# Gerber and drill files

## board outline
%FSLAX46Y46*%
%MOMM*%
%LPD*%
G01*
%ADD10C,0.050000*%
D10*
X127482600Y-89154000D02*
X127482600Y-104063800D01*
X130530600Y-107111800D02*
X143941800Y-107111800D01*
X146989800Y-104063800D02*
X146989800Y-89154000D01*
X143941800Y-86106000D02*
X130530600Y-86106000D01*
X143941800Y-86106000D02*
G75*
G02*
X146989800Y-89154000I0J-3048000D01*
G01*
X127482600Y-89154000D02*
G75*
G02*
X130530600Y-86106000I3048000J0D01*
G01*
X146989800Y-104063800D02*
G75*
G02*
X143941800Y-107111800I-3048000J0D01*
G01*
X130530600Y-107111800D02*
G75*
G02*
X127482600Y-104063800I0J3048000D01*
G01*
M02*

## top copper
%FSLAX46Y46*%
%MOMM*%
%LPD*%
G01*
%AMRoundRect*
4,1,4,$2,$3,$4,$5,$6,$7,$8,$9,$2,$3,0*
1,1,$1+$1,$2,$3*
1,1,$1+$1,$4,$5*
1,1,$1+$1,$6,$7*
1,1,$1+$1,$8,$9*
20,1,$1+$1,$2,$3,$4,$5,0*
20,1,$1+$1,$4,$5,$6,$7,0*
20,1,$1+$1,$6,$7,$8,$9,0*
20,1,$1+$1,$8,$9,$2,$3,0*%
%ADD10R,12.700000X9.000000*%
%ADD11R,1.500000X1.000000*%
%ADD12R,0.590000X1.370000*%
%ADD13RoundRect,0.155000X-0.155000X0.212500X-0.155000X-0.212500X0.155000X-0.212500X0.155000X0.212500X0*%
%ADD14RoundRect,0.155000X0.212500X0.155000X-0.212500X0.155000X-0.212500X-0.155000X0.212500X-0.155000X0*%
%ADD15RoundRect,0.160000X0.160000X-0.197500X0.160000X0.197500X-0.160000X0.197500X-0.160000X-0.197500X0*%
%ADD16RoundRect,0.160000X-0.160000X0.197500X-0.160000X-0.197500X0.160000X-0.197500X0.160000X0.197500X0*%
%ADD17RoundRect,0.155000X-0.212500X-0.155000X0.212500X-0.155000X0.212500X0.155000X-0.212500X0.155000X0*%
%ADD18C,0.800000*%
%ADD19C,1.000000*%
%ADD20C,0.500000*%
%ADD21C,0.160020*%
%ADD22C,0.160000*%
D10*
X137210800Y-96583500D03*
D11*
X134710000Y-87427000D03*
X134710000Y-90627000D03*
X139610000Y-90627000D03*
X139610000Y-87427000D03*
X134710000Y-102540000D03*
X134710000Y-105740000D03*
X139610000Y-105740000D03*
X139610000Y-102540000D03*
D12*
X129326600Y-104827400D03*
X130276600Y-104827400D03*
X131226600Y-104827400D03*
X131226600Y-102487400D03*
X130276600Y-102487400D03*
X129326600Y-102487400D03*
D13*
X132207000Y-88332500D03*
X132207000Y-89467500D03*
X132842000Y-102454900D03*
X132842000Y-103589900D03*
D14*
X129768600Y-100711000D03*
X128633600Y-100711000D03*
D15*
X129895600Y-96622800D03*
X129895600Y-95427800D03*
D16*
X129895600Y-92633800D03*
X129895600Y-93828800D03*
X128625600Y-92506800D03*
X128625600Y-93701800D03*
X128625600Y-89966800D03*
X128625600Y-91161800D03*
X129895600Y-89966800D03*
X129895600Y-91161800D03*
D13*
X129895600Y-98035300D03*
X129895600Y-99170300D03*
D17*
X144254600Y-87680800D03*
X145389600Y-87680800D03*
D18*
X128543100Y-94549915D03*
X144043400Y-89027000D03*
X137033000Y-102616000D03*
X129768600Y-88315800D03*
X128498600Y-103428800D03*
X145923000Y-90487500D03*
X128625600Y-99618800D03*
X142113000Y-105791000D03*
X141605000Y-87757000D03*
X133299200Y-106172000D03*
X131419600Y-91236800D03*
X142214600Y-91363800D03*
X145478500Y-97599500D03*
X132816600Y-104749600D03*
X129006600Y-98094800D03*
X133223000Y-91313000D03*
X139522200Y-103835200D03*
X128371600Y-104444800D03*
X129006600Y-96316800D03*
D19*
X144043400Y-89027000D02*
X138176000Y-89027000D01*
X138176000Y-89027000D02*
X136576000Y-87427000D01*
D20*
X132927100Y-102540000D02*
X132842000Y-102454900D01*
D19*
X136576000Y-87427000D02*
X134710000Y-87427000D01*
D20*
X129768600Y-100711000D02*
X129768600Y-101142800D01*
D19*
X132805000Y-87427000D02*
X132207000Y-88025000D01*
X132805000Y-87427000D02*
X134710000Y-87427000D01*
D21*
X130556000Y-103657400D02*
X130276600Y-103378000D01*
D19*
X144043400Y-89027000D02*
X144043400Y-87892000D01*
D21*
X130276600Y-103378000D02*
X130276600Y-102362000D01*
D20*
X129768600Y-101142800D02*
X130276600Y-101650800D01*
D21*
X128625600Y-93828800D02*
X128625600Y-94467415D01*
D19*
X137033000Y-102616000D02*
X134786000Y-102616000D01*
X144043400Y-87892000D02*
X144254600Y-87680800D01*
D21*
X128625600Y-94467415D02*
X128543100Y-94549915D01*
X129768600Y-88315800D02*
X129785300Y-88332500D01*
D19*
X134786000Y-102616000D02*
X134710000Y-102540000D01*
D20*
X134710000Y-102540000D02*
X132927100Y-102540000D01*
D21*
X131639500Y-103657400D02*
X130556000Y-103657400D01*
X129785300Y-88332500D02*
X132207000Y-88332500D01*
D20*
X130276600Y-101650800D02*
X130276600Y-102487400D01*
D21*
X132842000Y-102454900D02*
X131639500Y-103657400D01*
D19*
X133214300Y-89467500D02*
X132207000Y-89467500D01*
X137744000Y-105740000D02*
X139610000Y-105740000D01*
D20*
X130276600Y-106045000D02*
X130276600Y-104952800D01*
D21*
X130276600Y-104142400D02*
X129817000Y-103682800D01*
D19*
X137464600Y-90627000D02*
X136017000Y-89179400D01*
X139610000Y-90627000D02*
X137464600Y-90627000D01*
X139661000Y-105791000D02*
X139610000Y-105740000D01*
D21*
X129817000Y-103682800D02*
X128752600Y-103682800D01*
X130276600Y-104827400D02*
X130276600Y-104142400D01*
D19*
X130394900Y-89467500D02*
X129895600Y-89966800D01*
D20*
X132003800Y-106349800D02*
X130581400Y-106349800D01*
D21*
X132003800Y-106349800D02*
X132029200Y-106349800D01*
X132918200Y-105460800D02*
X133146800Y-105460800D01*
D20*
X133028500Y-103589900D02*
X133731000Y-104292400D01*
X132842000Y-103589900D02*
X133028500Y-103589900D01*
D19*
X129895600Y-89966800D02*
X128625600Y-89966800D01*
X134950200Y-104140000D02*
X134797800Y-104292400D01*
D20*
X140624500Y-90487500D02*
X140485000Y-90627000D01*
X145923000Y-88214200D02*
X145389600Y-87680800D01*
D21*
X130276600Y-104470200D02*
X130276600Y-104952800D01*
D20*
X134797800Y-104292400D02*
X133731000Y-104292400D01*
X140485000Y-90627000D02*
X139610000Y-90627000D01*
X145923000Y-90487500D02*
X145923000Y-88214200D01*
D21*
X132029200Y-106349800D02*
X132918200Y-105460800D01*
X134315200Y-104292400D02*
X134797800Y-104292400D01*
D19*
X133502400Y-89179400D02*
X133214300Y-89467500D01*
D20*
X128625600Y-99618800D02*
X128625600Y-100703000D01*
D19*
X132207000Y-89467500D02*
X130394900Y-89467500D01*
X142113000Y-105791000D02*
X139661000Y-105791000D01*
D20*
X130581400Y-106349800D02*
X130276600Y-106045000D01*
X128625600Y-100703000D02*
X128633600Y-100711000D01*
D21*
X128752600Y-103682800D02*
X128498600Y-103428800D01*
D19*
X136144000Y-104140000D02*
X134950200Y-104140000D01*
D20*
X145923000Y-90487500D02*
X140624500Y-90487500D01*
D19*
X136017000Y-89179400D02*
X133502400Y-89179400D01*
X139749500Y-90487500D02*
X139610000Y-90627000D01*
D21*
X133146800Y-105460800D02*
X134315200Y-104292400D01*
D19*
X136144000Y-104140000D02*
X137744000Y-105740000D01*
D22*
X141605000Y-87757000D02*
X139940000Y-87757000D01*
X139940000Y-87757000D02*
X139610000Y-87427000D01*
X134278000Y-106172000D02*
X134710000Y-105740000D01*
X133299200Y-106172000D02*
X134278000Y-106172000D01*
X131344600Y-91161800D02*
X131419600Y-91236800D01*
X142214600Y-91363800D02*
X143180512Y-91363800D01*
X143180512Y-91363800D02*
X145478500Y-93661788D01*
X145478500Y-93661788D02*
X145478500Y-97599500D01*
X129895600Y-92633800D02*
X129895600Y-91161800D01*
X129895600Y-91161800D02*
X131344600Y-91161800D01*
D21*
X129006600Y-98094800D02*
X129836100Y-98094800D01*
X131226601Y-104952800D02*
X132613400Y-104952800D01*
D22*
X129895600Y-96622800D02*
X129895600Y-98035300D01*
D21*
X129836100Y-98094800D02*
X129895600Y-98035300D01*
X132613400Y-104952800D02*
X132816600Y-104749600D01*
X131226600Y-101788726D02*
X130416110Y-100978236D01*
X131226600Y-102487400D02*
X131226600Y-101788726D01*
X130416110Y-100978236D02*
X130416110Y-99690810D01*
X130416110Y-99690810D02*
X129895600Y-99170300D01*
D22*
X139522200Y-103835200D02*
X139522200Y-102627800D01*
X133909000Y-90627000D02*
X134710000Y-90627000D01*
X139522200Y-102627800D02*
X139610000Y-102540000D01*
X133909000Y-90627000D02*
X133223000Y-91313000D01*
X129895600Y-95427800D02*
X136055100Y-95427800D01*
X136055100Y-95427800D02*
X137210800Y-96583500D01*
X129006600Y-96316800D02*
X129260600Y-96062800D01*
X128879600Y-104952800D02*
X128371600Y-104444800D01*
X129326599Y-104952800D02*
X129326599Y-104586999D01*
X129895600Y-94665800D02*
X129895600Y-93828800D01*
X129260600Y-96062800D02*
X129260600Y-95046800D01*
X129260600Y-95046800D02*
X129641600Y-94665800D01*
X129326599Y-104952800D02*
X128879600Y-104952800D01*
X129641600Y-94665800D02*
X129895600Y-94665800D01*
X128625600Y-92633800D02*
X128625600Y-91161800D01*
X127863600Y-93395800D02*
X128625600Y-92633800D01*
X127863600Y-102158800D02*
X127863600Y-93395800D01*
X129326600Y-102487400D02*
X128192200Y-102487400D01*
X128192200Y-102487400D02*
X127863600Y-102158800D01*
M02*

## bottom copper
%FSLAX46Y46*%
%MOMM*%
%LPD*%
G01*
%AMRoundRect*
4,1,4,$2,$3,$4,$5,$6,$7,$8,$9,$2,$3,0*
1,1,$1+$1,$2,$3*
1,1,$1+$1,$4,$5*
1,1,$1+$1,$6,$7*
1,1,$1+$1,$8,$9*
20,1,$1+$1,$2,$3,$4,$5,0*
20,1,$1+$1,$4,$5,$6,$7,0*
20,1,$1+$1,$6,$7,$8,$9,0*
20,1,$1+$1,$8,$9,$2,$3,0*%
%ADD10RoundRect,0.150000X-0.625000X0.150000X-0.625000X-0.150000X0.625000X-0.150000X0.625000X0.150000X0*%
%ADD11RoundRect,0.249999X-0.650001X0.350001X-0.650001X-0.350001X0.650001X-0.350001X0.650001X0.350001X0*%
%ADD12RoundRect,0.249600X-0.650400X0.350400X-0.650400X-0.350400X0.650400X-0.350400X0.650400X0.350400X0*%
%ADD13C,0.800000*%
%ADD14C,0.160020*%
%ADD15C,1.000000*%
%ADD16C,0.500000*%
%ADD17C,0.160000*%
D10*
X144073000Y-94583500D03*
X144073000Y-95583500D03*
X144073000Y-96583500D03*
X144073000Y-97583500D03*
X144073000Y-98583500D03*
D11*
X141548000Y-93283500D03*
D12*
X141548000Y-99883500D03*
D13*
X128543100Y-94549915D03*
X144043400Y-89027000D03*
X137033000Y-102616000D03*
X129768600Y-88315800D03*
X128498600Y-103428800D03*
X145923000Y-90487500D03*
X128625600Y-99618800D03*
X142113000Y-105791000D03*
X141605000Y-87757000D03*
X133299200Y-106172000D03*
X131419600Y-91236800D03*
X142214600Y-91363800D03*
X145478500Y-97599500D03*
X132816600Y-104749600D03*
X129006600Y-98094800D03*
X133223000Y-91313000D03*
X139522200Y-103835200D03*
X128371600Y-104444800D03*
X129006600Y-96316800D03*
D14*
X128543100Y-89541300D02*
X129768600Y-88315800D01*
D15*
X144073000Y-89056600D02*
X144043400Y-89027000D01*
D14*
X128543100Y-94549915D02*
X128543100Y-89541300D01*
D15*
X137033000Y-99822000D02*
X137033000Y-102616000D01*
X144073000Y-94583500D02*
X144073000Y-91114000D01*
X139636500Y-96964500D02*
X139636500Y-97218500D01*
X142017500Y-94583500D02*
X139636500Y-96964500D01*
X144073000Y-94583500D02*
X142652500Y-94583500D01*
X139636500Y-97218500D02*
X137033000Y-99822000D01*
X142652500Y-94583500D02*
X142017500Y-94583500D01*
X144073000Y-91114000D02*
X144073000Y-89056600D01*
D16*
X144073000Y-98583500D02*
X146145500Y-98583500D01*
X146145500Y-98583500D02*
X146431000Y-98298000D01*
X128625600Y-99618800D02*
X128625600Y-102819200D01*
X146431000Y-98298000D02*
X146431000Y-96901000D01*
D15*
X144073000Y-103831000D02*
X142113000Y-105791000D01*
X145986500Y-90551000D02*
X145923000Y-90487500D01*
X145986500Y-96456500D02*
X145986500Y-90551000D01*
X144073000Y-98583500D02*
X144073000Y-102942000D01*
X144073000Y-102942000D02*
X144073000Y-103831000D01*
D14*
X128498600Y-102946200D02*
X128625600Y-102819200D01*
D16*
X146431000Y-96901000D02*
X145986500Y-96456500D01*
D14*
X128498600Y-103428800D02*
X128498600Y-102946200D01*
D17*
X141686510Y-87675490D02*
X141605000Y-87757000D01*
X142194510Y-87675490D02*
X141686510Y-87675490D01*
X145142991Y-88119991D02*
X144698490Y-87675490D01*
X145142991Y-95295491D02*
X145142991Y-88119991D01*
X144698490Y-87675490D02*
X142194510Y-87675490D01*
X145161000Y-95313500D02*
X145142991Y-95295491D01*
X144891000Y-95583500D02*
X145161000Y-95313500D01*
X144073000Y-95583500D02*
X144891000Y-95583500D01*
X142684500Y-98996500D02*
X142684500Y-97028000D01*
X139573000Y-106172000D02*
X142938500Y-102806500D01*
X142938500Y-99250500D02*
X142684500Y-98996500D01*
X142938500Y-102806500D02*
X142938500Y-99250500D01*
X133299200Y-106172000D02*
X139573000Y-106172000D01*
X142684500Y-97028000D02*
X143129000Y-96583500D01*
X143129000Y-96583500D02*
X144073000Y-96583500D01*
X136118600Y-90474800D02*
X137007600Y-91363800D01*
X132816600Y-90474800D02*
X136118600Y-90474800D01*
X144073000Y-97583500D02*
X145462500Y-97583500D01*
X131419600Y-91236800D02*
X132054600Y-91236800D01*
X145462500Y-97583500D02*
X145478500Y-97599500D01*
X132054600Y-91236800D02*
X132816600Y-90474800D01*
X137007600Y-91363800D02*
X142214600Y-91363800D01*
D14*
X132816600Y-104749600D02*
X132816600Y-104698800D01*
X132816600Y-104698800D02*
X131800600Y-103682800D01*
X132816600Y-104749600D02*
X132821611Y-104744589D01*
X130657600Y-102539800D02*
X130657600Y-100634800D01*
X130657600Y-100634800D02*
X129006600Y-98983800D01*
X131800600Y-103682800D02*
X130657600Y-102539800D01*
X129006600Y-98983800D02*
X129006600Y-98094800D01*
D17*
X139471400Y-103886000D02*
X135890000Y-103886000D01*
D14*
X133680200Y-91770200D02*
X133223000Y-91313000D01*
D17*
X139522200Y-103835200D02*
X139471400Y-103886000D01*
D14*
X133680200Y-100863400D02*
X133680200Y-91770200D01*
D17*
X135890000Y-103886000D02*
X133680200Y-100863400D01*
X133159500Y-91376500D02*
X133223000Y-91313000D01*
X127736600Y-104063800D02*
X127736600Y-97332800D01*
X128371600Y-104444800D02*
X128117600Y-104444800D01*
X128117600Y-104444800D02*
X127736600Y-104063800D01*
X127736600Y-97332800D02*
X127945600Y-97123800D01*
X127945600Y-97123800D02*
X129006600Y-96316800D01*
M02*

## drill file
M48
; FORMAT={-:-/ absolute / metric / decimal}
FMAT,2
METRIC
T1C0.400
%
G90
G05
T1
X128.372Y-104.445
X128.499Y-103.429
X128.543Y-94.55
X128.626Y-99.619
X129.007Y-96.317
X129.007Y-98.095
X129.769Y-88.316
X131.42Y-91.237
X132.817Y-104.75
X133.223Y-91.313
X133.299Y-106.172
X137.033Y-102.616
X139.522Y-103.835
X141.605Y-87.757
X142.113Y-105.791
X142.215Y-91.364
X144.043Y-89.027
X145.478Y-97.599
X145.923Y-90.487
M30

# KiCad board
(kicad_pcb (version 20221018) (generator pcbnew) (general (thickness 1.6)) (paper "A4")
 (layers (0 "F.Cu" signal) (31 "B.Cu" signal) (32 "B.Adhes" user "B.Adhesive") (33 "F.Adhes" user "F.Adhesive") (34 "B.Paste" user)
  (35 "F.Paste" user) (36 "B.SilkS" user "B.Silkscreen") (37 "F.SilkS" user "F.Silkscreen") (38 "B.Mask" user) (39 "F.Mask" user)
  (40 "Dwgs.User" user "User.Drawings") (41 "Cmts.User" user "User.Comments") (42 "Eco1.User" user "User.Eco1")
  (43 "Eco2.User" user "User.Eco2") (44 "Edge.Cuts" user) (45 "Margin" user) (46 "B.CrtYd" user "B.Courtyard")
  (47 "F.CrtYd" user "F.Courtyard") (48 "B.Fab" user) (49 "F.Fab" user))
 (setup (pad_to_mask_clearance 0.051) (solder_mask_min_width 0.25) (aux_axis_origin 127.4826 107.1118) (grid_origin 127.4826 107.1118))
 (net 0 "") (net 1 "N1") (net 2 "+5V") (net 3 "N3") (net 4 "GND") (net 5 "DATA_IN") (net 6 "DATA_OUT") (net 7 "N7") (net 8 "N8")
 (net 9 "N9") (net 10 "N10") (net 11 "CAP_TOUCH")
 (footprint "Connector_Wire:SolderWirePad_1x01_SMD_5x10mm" (layer "F.Cu") (at 136.0805 96.647)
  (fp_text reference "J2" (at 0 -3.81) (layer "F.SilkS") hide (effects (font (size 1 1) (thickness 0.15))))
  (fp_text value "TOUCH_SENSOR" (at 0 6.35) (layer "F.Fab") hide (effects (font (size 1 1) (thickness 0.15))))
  (pad "1" smd rect (at 1.1303 -0.0635) (size 12.7 9) (layers "F.Cu" "F.Mask") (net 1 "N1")))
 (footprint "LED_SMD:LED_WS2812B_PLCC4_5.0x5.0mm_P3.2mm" (layer "F.Cu") (at 137.16 89.027)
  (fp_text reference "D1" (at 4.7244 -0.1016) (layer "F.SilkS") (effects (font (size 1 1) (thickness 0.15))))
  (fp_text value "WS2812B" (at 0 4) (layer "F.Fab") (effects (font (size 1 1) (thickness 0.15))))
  (pad "1" smd rect (at -2.45 -1.6) (size 1.5 1) (layers "F.Cu" "F.Paste" "F.Mask") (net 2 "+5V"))
  (pad "2" smd rect (at -2.45 1.6) (size 1.5 1) (layers "F.Cu" "F.Paste" "F.Mask") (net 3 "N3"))
  (pad "3" smd rect (at 2.45 1.6) (size 1.5 1) (layers "F.Cu" "F.Paste" "F.Mask") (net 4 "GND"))
  (pad "4" smd rect (at 2.45 -1.6) (size 1.5 1) (layers "F.Cu" "F.Paste" "F.Mask") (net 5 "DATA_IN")))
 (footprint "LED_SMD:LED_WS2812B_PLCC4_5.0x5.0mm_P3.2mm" (layer "F.Cu") (at 137.16 104.14)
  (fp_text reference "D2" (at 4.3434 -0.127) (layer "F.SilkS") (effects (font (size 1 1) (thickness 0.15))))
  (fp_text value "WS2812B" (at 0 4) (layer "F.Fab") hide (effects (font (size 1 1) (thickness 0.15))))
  (pad "1" smd rect (at -2.45 -1.6) (size 1.5 1) (layers "F.Cu" "F.Paste" "F.Mask") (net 2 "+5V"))
  (pad "2" smd rect (at -2.45 1.6) (size 1.5 1) (layers "F.Cu" "F.Paste" "F.Mask") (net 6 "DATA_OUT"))
  (pad "3" smd rect (at 2.45 1.6) (size 1.5 1) (layers "F.Cu" "F.Paste" "F.Mask") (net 4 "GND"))
  (pad "4" smd rect (at 2.45 -1.6) (size 1.5 1) (layers "F.Cu" "F.Paste" "F.Mask") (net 3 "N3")))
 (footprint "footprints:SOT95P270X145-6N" (layer "F.Cu") (at 130.2766 103.6574 90)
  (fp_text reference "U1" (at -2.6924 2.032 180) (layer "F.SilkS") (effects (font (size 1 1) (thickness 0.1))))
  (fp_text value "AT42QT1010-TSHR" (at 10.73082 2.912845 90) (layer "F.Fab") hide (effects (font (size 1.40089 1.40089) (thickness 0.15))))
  (pad "1" smd rect (at -1.17 -0.95 90) (size 1.37 0.59) (layers "F.Cu" "F.Paste" "F.Mask") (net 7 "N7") (solder_mask_margin 0.102))
  (pad "2" smd rect (at -1.17 0 90) (size 1.37 0.59) (layers "F.Cu" "F.Paste" "F.Mask") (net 4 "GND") (solder_mask_margin 0.102))
  (pad "3" smd rect (at -1.17 0.95 90) (size 1.37 0.59) (layers "F.Cu" "F.Paste" "F.Mask") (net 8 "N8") (solder_mask_margin 0.102))
  (pad "4" smd rect (at 1.17 0.95 90) (size 1.37 0.59) (layers "F.Cu" "F.Paste" "F.Mask") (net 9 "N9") (solder_mask_margin 0.102))
  (pad "5" smd rect (at 1.17 0 90) (size 1.37 0.59) (layers "F.Cu" "F.Paste" "F.Mask") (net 2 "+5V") (solder_mask_margin 0.102))
  (pad "6" smd rect (at 1.17 -0.95 90) (size 1.37 0.59) (layers "F.Cu" "F.Paste" "F.Mask") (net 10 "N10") (solder_mask_margin 0.102)))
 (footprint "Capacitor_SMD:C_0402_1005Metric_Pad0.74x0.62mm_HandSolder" (layer "F.Cu") (at 132.207 88.9 -90)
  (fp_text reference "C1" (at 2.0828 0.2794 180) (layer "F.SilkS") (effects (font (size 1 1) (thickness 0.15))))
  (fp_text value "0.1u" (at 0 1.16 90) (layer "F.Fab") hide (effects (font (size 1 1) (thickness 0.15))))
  (pad "1" smd roundrect (at -0.5675 0 270) (size 0.735 0.62) (layers "F.Cu" "F.Paste" "F.Mask") (roundrect_rratio 0.25) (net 2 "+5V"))
  (pad "2" smd roundrect (at 0.5675 0 270) (size 0.735 0.62) (layers "F.Cu" "F.Paste" "F.Mask") (roundrect_rratio 0.25) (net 4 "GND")))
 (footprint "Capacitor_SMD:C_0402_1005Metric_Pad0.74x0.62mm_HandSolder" (layer "F.Cu") (at 132.842 103.0224 -90)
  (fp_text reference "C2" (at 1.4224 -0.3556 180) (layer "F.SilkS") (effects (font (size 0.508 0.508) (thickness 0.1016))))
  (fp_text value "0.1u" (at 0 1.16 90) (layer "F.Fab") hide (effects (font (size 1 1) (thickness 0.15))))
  (pad "1" smd roundrect (at -0.5675 0 270) (size 0.735 0.62) (layers "F.Cu" "F.Paste" "F.Mask") (roundrect_rratio 0.25) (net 2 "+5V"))
  (pad "2" smd roundrect (at 0.5675 0 270) (size 0.735 0.62) (layers "F.Cu" "F.Paste" "F.Mask") (roundrect_rratio 0.25) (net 4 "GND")))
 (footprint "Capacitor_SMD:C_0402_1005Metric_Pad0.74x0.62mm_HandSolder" (layer "F.Cu") (at 129.2011 100.711 180)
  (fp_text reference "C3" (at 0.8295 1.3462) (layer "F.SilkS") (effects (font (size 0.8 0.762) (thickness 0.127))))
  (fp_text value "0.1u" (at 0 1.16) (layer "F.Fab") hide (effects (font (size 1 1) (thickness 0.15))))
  (pad "1" smd roundrect (at -0.5675 0 180) (size 0.735 0.62) (layers "F.Cu" "F.Paste" "F.Mask") (roundrect_rratio 0.25) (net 2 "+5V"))
  (pad "2" smd roundrect (at 0.5675 0 180) (size 0.735 0.62) (layers "F.Cu" "F.Paste" "F.Mask") (roundrect_rratio 0.25) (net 4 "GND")))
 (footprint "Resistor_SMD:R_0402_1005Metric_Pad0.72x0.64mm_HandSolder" (layer "F.Cu") (at 129.8956 96.0253 90)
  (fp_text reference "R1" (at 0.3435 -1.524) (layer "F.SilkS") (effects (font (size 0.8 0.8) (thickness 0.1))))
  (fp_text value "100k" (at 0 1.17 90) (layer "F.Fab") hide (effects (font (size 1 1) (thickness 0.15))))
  (pad "1" smd roundrect (at -0.5975 0 90) (size 0.715 0.64) (layers "F.Cu" "F.Paste" "F.Mask") (roundrect_rratio 0.25) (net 8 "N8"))
  (pad "2" smd roundrect (at 0.5975 0 90) (size 0.715 0.64) (layers "F.Cu" "F.Paste" "F.Mask") (roundrect_rratio 0.25) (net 1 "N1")))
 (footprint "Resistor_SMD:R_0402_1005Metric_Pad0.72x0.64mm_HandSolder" (layer "F.Cu") (at 129.8956 93.2313 -90)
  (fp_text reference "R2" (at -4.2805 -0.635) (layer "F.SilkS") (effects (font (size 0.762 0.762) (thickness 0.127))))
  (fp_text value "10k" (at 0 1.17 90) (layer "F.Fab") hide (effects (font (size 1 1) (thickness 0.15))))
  (pad "1" smd roundrect (at -0.5975 0 270) (size 0.715 0.64) (layers "F.Cu" "F.Paste" "F.Mask") (roundrect_rratio 0.25)
   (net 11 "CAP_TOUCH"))
  (pad "2" smd roundrect (at 0.5975 0 270) (size 0.715 0.64) (layers "F.Cu" "F.Paste" "F.Mask") (roundrect_rratio 0.25) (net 7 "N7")))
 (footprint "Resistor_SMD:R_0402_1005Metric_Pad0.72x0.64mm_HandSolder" (layer "F.Cu") (at 128.6256 93.1043 -90)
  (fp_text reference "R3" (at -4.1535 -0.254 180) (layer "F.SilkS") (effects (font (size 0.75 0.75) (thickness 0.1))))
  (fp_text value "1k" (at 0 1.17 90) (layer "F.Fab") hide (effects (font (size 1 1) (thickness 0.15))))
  (pad "1" smd roundrect (at -0.5975 0 270) (size 0.715 0.64) (layers "F.Cu" "F.Paste" "F.Mask") (roundrect_rratio 0.25) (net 10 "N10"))
  (pad "2" smd roundrect (at 0.5975 0 270) (size 0.715 0.64) (layers "F.Cu" "F.Paste" "F.Mask") (roundrect_rratio 0.25) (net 2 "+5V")))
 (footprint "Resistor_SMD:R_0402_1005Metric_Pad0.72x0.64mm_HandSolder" (layer "F.Cu") (at 128.6256 90.5643 -90)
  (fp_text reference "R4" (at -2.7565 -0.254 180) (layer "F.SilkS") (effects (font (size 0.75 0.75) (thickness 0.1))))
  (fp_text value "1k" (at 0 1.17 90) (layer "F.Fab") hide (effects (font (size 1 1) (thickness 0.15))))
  (pad "1" smd roundrect (at -0.5975 0 270) (size 0.715 0.64) (layers "F.Cu" "F.Paste" "F.Mask") (roundrect_rratio 0.25) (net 4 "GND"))
  (pad "2" smd roundrect (at 0.5975 0 270) (size 0.715 0.64) (layers "F.Cu" "F.Paste" "F.Mask") (roundrect_rratio 0.25) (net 10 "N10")))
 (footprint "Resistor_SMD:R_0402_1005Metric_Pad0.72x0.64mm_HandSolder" (layer "F.Cu") (at 129.8956 90.5643 -90)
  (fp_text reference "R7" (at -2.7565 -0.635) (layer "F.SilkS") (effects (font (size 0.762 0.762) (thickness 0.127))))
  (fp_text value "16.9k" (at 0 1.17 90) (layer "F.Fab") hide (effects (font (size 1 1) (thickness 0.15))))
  (pad "1" smd roundrect (at -0.5975 0 270) (size 0.715 0.64) (layers "F.Cu" "F.Paste" "F.Mask") (roundrect_rratio 0.25) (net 4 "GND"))
  (pad "2" smd roundrect (at 0.5975 0 270) (size 0.715 0.64) (layers "F.Cu" "F.Paste" "F.Mask") (roundrect_rratio 0.25) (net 11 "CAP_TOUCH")))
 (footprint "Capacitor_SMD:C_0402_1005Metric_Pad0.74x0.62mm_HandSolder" (layer "F.Cu") (at 129.8956 98.6028 -90)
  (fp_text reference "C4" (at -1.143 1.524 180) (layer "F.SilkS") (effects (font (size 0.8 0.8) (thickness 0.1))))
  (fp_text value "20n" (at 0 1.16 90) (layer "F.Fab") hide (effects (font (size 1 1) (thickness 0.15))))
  (pad "1" smd roundrect (at -0.5675 0 270) (size 0.735 0.62) (layers "F.Cu" "F.Paste" "F.Mask") (roundrect_rratio 0.25) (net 8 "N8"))
  (pad "2" smd roundrect (at 0.5675 0 270) (size 0.735 0.62) (layers "F.Cu" "F.Paste" "F.Mask") (roundrect_rratio 0.25) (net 9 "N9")))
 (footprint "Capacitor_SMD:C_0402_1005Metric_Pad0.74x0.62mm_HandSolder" (layer "F.Cu") (at 144.8221 87.6808)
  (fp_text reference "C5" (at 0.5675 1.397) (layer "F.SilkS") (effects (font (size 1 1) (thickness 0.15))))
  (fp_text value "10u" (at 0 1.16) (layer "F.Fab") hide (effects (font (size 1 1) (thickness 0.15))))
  (pad "1" smd roundrect (at -0.5675 0) (size 0.735 0.62) (layers "F.Cu" "F.Paste" "F.Mask") (roundrect_rratio 0.25) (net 2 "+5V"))
  (pad "2" smd roundrect (at 0.5675 0) (size 0.735 0.62) (layers "F.Cu" "F.Paste" "F.Mask") (roundrect_rratio 0.25) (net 4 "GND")))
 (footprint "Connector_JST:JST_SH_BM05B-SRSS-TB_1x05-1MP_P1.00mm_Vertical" (layer "B.Cu") (at 142.748 96.5835 -90)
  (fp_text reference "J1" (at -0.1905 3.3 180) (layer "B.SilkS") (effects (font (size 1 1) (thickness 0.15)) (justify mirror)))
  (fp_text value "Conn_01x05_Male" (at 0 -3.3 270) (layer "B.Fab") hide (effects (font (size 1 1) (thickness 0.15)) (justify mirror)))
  (pad "1" smd roundrect (at -2 -1.325 270) (size 0.6 1.55) (layers "B.Cu" "B.Mask") (roundrect_rratio 0.25) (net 2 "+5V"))
  (pad "2" smd roundrect (at -1 -1.325 270) (size 0.6 1.55) (layers "B.Cu" "B.Mask") (roundrect_rratio 0.25) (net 5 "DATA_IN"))
  (pad "3" smd roundrect (at 0 -1.325 270) (size 0.6 1.55) (layers "B.Cu" "B.Mask") (roundrect_rratio 0.25) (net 6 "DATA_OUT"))
  (pad "4" smd roundrect (at 1 -1.325 270) (size 0.6 1.55) (layers "B.Cu" "B.Mask") (roundrect_rratio 0.25) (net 11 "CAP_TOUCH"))
  (pad "5" smd roundrect (at 2 -1.325 270) (size 0.6 1.55) (layers "B.Cu" "B.Mask") (roundrect_rratio 0.25) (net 4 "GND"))
  (pad "MP" smd roundrect (at -3.3 1.2 270) (size 1.2 1.8) (layers "B.Cu" "B.Paste" "B.Mask") (roundrect_rratio 0.2083325))
  (pad "MP" smd roundrect (at 3.3 1.2 270) (size 1.2 1.8) (layers "B.Cu" "B.Mask") (roundrect_rratio 0.208)))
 (gr_line (start 127.4826 89.154) (end 127.4826 104.0638) (stroke (width 0.05) (type solid)) (layer "Edge.Cuts"))
 (gr_line (start 130.5306 107.1118) (end 143.9418 107.1118) (stroke (width 0.05) (type solid)) (layer "Edge.Cuts"))
 (gr_line (start 146.9898 104.0638) (end 146.9898 89.154) (stroke (width 0.05) (type solid)) (layer "Edge.Cuts"))
 (gr_line (start 143.9418 86.106) (end 130.5306 86.106) (stroke (width 0.05) (type solid)) (layer "Edge.Cuts"))
 (gr_arc (start 143.9418 86.106) (mid 146.097061 86.998739) (end 146.9898 89.154) (stroke (width 0.05) (type solid)) (layer "Edge.Cuts"))
 (gr_arc (start 127.4826 89.154) (mid 128.375339 86.998739) (end 130.5306 86.106) (stroke (width 0.05) (type solid)) (layer "Edge.Cuts"))
 (gr_arc (start 146.9898 104.0638) (mid 146.097061 106.219061) (end 143.9418 107.1118) (stroke (width 0.05) (type solid))
  (layer "Edge.Cuts"))
 (gr_arc (start 130.5306 107.1118) (mid 128.375339 106.219061) (end 127.4826 104.0638) (stroke (width 0.05) (type solid))
  (layer "Edge.Cuts"))
 (segment (start 144.0434 89.027) (end 138.176 89.027) (width 1) (layer "F.Cu") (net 2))
 (segment (start 138.176 89.027) (end 136.576 87.427) (width 1) (layer "F.Cu") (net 2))
 (segment (start 132.9271 102.54) (end 132.842 102.4549) (width 0.5) (layer "F.Cu") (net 2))
 (segment (start 136.576 87.427) (end 134.71 87.427) (width 1) (layer "F.Cu") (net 2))
 (segment (start 129.7686 100.711) (end 129.7686 101.1428) (width 0.5) (layer "F.Cu") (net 2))
 (segment (start 132.805 87.427) (end 132.207 88.025) (width 1) (layer "F.Cu") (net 2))
 (segment (start 132.805 87.427) (end 134.71 87.427) (width 1) (layer "F.Cu") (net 2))
 (segment (start 130.556 103.6574) (end 130.2766 103.378) (width 0.16002) (layer "F.Cu") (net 2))
 (segment (start 144.0434 89.027) (end 144.0434 87.892) (width 1) (layer "F.Cu") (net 2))
 (segment (start 130.2766 103.378) (end 130.2766 102.362) (width 0.16002) (layer "F.Cu") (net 2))
 (segment (start 129.7686 101.1428) (end 130.2766 101.6508) (width 0.5) (layer "F.Cu") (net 2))
 (segment (start 128.6256 93.8288) (end 128.6256 94.467415) (width 0.16002) (layer "F.Cu") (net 2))
 (segment (start 137.033 102.616) (end 134.786 102.616) (width 1) (layer "F.Cu") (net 2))
 (segment (start 144.0434 87.892) (end 144.2546 87.6808) (width 1) (layer "F.Cu") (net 2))
 (segment (start 128.6256 94.467415) (end 128.5431 94.549915) (width 0.16002) (layer "F.Cu") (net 2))
 (segment (start 129.7686 88.3158) (end 129.7853 88.3325) (width 0.16002) (layer "F.Cu") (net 2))
 (segment (start 134.786 102.616) (end 134.71 102.54) (width 1) (layer "F.Cu") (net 2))
 (segment (start 134.71 102.54) (end 132.9271 102.54) (width 0.5) (layer "F.Cu") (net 2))
 (segment (start 131.6395 103.6574) (end 130.556 103.6574) (width 0.16002) (layer "F.Cu") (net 2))
 (segment (start 129.7853 88.3325) (end 132.207 88.3325) (width 0.16002) (layer "F.Cu") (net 2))
 (segment (start 130.2766 101.6508) (end 130.2766 102.4874) (width 0.5) (layer "F.Cu") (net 2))
 (segment (start 132.842 102.4549) (end 131.6395 103.6574) (width 0.16002) (layer "F.Cu") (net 2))
 (via (at 128.5431 94.549915) (size 0.8) (drill 0.4) (layers "F.Cu" "B.Cu") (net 2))
 (via (at 144.0434 89.027) (size 0.8) (drill 0.4) (layers "F.Cu" "B.Cu") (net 2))
 (via (at 137.033 102.616) (size 0.8) (drill 0.4) (layers "F.Cu" "B.Cu") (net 2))
 (via (at 129.7686 88.3158) (size 0.8) (drill 0.4) (layers "F.Cu" "B.Cu") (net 2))
 (segment (start 128.5431 89.5413) (end 129.7686 88.3158) (width 0.16002) (layer "B.Cu") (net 2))
 (segment (start 144.073 89.0566) (end 144.0434 89.027) (width 1) (layer "B.Cu") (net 2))
 (segment (start 128.5431 94.549915) (end 128.5431 89.5413) (width 0.16002) (layer "B.Cu") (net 2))
 (segment (start 137.033 99.822) (end 137.033 102.616) (width 1) (layer "B.Cu") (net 2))
 (segment (start 144.073 94.5835) (end 144.073 91.114) (width 1) (layer "B.Cu") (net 2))
 (segment (start 139.6365 96.9645) (end 139.6365 97.2185) (width 1) (layer "B.Cu") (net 2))
 (segment (start 142.0175 94.5835) (end 139.6365 96.9645) (width 1) (layer "B.Cu") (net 2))
 (segment (start 144.073 94.5835) (end 142.6525 94.5835) (width 1) (layer "B.Cu") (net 2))
 (segment (start 139.6365 97.2185) (end 137.033 99.822) (width 1) (layer "B.Cu") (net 2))
 (segment (start 142.6525 94.5835) (end 142.0175 94.5835) (width 1) (layer "B.Cu") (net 2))
 (segment (start 144.073 91.114) (end 144.073 89.0566) (width 1) (layer "B.Cu") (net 2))
 (segment (start 133.2143 89.4675) (end 132.207 89.4675) (width 1) (layer "F.Cu") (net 4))
 (segment (start 137.744 105.74) (end 139.61 105.74) (width 1) (layer "F.Cu") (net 4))
 (segment (start 130.2766 106.045) (end 130.2766 104.9528) (width 0.5) (layer "F.Cu") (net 4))
 (segment (start 130.2766 104.1424) (end 129.817 103.6828) (width 0.16002) (layer "F.Cu") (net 4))
 (segment (start 137.4646 90.627) (end 136.017 89.1794) (width 1) (layer "F.Cu") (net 4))
 (segment (start 139.61 90.627) (end 137.4646 90.627) (width 1) (layer "F.Cu") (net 4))
 (segment (start 139.661 105.791) (end 139.61 105.74) (width 1) (layer "F.Cu") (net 4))
 (segment (start 129.817 103.6828) (end 128.7526 103.6828) (width 0.16002) (layer "F.Cu") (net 4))
 (segment (start 130.2766 104.8274) (end 130.2766 104.1424) (width 0.16002) (layer "F.Cu") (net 4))
 (segment (start 130.3949 89.4675) (end 129.8956 89.9668) (width 1) (layer "F.Cu") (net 4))
 (segment (start 132.0038 106.3498) (end 130.5814 106.3498) (width 0.5) (layer "F.Cu") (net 4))
 (segment (start 132.0038 106.3498) (end 132.0292 106.3498) (width 0.16002) (layer "F.Cu") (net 4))
 (segment (start 132.9182 105.4608) (end 133.1468 105.4608) (width 0.16002) (layer "F.Cu") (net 4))
 (segment (start 133.0285 103.5899) (end 133.731 104.2924) (width 0.5) (layer "F.Cu") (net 4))
 (segment (start 132.842 103.5899) (end 133.0285 103.5899) (width 0.5) (layer "F.Cu") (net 4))
 (segment (start 129.8956 89.9668) (end 128.6256 89.9668) (width 1) (layer "F.Cu") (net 4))
 (segment (start 134.9502 104.14) (end 134.7978 104.2924) (width 1) (layer "F.Cu") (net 4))
 (segment (start 140.6245 90.4875) (end 140.485 90.627) (width 0.5) (layer "F.Cu") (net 4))
 (segment (start 145.923 88.2142) (end 145.3896 87.6808) (width 0.5) (layer "F.Cu") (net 4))
 (segment (start 130.2766 104.4702) (end 130.2766 104.9528) (width 0.16002) (layer "F.Cu") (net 4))
 (segment (start 134.7978 104.2924) (end 133.731 104.2924) (width 0.5) (layer "F.Cu") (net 4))
 (segment (start 140.485 90.627) (end 139.61 90.627) (width 0.5) (layer "F.Cu") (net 4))
 (segment (start 145.923 90.4875) (end 145.923 88.2142) (width 0.5) (layer "F.Cu") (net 4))
 (segment (start 132.0292 106.3498) (end 132.9182 105.4608) (width 0.16002) (layer "F.Cu") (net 4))
 (segment (start 134.3152 104.2924) (end 134.7978 104.2924) (width 0.16002) (layer "F.Cu") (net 4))
 (segment (start 133.5024 89.1794) (end 133.2143 89.4675) (width 1) (layer "F.Cu") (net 4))
 (segment (start 128.6256 99.6188) (end 128.6256 100.703) (width 0.5) (layer "F.Cu") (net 4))
 (segment (start 132.207 89.4675) (end 130.3949 89.4675) (width 1) (layer "F.Cu") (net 4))
 (segment (start 142.113 105.791) (end 139.661 105.791) (width 1) (layer "F.Cu") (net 4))
 (segment (start 130.5814 106.3498) (end 130.2766 106.045) (width 0.5) (layer "F.Cu") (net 4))
 (segment (start 128.6256 100.703) (end 128.6336 100.711) (width 0.5) (layer "F.Cu") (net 4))
 (segment (start 128.7526 103.6828) (end 128.4986 103.4288) (width 0.16002) (layer "F.Cu") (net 4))
 (segment (start 136.144 104.14) (end 134.9502 104.14) (width 1) (layer "F.Cu") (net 4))
 (segment (start 145.923 90.4875) (end 140.6245 90.4875) (width 0.5) (layer "F.Cu") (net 4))
 (segment (start 136.017 89.1794) (end 133.5024 89.1794) (width 1) (layer "F.Cu") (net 4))
 (segment (start 139.7495 90.4875) (end 139.61 90.627) (width 1) (layer "F.Cu") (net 4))
 (segment (start 133.1468 105.4608) (end 134.3152 104.2924) (width 0.16002) (layer "F.Cu") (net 4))
 (segment (start 136.144 104.14) (end 137.744 105.74) (width 1) (layer "F.Cu") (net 4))
 (via (at 128.4986 103.4288) (size 0.8) (drill 0.4) (layers "F.Cu" "B.Cu") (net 4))
 (via (at 145.923 90.4875) (size 0.8) (drill 0.4) (layers "F.Cu" "B.Cu") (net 4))
 (via (at 128.6256 99.6188) (size 0.8) (drill 0.4) (layers "F.Cu" "B.Cu") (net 4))
 (via (at 142.113 105.791) (size 0.8) (drill 0.4) (layers "F.Cu" "B.Cu") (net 4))
 (segment (start 144.073 98.5835) (end 146.1455 98.5835) (width 0.5) (layer "B.Cu") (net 4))
 (segment (start 146.1455 98.5835) (end 146.431 98.298) (width 0.5) (layer "B.Cu") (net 4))
 (segment (start 128.6256 99.6188) (end 128.6256 102.8192) (width 0.5) (layer "B.Cu") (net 4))
 (segment (start 146.431 98.298) (end 146.431 96.901) (width 0.5) (layer "B.Cu") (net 4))
 (segment (start 144.073 103.831) (end 142.113 105.791) (width 1) (layer "B.Cu") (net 4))
 (segment (start 145.9865 90.551) (end 145.923 90.4875) (width 1) (layer "B.Cu") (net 4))
 (segment (start 145.9865 96.4565) (end 145.9865 90.551) (width 1) (layer "B.Cu") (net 4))
 (segment (start 144.073 98.5835) (end 144.073 102.942) (width 1) (layer "B.Cu") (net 4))
 (segment (start 144.073 102.942) (end 144.073 103.831) (width 1) (layer "B.Cu") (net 4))
 (segment (start 128.4986 102.9462) (end 128.6256 102.8192) (width 0.16002) (layer "B.Cu") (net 4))
 (segment (start 146.431 96.901) (end 145.9865 96.4565) (width 0.5) (layer "B.Cu") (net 4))
 (segment (start 128.4986 103.4288) (end 128.4986 102.9462) (width 0.16002) (layer "B.Cu") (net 4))
 (segment (start 141.605 87.757) (end 139.94 87.757) (width 0.16) (layer "F.Cu") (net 5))
 (segment (start 139.94 87.757) (end 139.61 87.427) (width 0.16) (layer "F.Cu") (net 5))
 (via (at 141.605 87.757) (size 0.8) (drill 0.4) (layers "F.Cu" "B.Cu") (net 5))
 (segment (start 141.68651 87.67549) (end 141.605 87.757) (width 0.16) (layer "B.Cu") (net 5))
 (segment (start 142.19451 87.67549) (end 141.68651 87.67549) (width 0.16) (layer "B.Cu") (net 5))
 (segment (start 145.142991 88.119991) (end 144.69849 87.67549) (width 0.16) (layer "B.Cu") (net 5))
 (segment (start 145.142991 95.295491) (end 145.142991 88.119991) (width 0.16) (layer "B.Cu") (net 5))
 (segment (start 144.69849 87.67549) (end 142.19451 87.67549) (width 0.16) (layer "B.Cu") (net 5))
 (segment (start 145.161 95.3135) (end 145.142991 95.295491) (width 0.16) (layer "B.Cu") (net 5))
 (segment (start 144.891 95.5835) (end 145.161 95.3135) (width 0.16) (layer "B.Cu") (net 5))
 (segment (start 144.073 95.5835) (end 144.891 95.5835) (width 0.16) (layer "B.Cu") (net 5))
 (segment (start 134.278 106.172) (end 134.71 105.74) (width 0.16) (layer "F.Cu") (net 6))
 (segment (start 133.2992 106.172) (end 134.278 106.172) (width 0.16) (layer "F.Cu") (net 6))
 (via (at 133.2992 106.172) (size 0.8) (drill 0.4) (layers "F.Cu" "B.Cu") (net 6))
 (segment (start 142.6845 98.9965) (end 142.6845 97.028) (width 0.16) (layer "B.Cu") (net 6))
 (segment (start 139.573 106.172) (end 142.9385 102.8065) (width 0.16) (layer "B.Cu") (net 6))
 (segment (start 142.9385 99.2505) (end 142.6845 98.9965) (width 0.16) (layer "B.Cu") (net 6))
 (segment (start 142.9385 102.8065) (end 142.9385 99.2505) (width 0.16) (layer "B.Cu") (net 6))
 (segment (start 133.2992 106.172) (end 139.573 106.172) (width 0.16) (layer "B.Cu") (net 6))
 (segment (start 142.6845 97.028) (end 143.129 96.5835) (width 0.16) (layer "B.Cu") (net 6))
 (segment (start 143.129 96.5835) (end 144.073 96.5835) (width 0.16) (layer "B.Cu") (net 6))
 (segment (start 131.3446 91.1618) (end 131.4196 91.2368) (width 0.16) (layer "F.Cu") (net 11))
 (segment (start 142.2146 91.3638) (end 143.180512 91.3638) (width 0.16) (layer "F.Cu") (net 11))
 (segment (start 143.180512 91.3638) (end 145.4785 93.661788) (width 0.16) (layer "F.Cu") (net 11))
 (segment (start 145.4785 93.661788) (end 145.4785 97.5995) (width 0.16) (layer "F.Cu") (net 11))
 (segment (start 129.8956 92.6338) (end 129.8956 91.1618) (width 0.16) (layer "F.Cu") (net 11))
 (segment (start 129.8956 91.1618) (end 131.3446 91.1618) (width 0.16) (layer "F.Cu") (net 11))
 (via (at 131.4196 91.2368) (size 0.8) (drill 0.4) (layers "F.Cu" "B.Cu") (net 11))
 (via (at 142.2146 91.3638) (size 0.8) (drill 0.4) (layers "F.Cu" "B.Cu") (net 11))
 (via (at 145.4785 97.5995) (size 0.8) (drill 0.4) (layers "F.Cu" "B.Cu") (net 11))
 (segment (start 136.1186 90.4748) (end 137.0076 91.3638) (width 0.16) (layer "B.Cu") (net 11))
 (segment (start 132.8166 90.4748) (end 136.1186 90.4748) (width 0.16) (layer "B.Cu") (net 11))
 (segment (start 144.073 97.5835) (end 145.4625 97.5835) (width 0.16) (layer "B.Cu") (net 11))
 (segment (start 131.4196 91.2368) (end 132.0546 91.2368) (width 0.16) (layer "B.Cu") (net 11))
 (segment (start 145.4625 97.5835) (end 145.4785 97.5995) (width 0.16) (layer "B.Cu") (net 11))
 (segment (start 132.0546 91.2368) (end 132.8166 90.4748) (width 0.16) (layer "B.Cu") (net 11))
 (segment (start 137.0076 91.3638) (end 142.2146 91.3638) (width 0.16) (layer "B.Cu") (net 11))
 (segment (start 129.0066 98.0948) (end 129.8361 98.0948) (width 0.16002) (layer "F.Cu") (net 8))
 (segment (start 131.226601 104.9528) (end 132.6134 104.9528) (width 0.16002) (layer "F.Cu") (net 8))
 (segment (start 129.8956 96.6228) (end 129.8956 98.0353) (width 0.16) (layer "F.Cu") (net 8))
 (segment (start 129.8361 98.0948) (end 129.8956 98.0353) (width 0.16002) (layer "F.Cu") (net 8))
 (segment (start 132.6134 104.9528) (end 132.8166 104.7496) (width 0.16002) (layer "F.Cu") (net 8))
 (via (at 132.8166 104.7496) (size 0.8) (drill 0.4) (layers "F.Cu" "B.Cu") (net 8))
 (via (at 129.0066 98.0948) (size 0.8) (drill 0.4) (layers "F.Cu" "B.Cu") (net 8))
 (segment (start 132.8166 104.7496) (end 132.8166 104.6988) (width 0.16002) (layer "B.Cu") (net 8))
 (segment (start 132.8166 104.6988) (end 131.8006 103.6828) (width 0.16002) (layer "B.Cu") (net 8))
 (segment (start 132.8166 104.7496) (end 132.821611 104.744589) (width 0.16002) (layer "B.Cu") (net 8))
 (segment (start 130.6576 102.5398) (end 130.6576 100.6348) (width 0.16002) (layer "B.Cu") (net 8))
 (segment (start 130.6576 100.6348) (end 129.0066 98.9838) (width 0.16002) (layer "B.Cu") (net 8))
 (segment (start 131.8006 103.6828) (end 130.6576 102.5398) (width 0.16002) (layer "B.Cu") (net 8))
 (segment (start 129.0066 98.9838) (end 129.0066 98.0948) (width 0.16002) (layer "B.Cu") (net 8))
 (segment (start 131.2266 101.788726) (end 130.41611 100.978236) (width 0.16002) (layer "F.Cu") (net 9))
 (segment (start 131.2266 102.4874) (end 131.2266 101.788726) (width 0.16002) (layer "F.Cu") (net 9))
 (segment (start 130.41611 100.978236) (end 130.41611 99.69081) (width 0.16002) (layer "F.Cu") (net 9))
 (segment (start 130.41611 99.69081) (end 129.8956 99.1703) (width 0.16002) (layer "F.Cu") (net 9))
 (segment (start 139.5222 103.8352) (end 139.5222 102.6278) (width 0.16) (layer "F.Cu") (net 3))
 (segment (start 133.909 90.627) (end 134.71 90.627) (width 0.16) (layer "F.Cu") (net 3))
 (segment (start 139.5222 102.6278) (end 139.61 102.54) (width 0.16) (layer "F.Cu") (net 3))
 (segment (start 133.909 90.627) (end 133.223 91.313) (width 0.16) (layer "F.Cu") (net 3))
 (via (at 133.223 91.313) (size 0.8) (drill 0.4) (layers "F.Cu" "B.Cu") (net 3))
 (via (at 139.5222 103.8352) (size 0.8) (drill 0.4) (layers "F.Cu" "B.Cu") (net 3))
 (segment (start 139.4714 103.886) (end 135.89 103.886) (width 0.16) (layer "B.Cu") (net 3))
 (segment (start 133.6802 91.7702) (end 133.223 91.313) (width 0.16002) (layer "B.Cu") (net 3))
 (segment (start 139.5222 103.8352) (end 139.4714 103.886) (width 0.16) (layer "B.Cu") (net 3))
 (segment (start 133.6802 100.8634) (end 133.6802 91.7702) (width 0.16002) (layer "B.Cu") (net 3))
 (segment (start 135.89 103.886) (end 133.6802 100.8634) (width 0.16) (layer "B.Cu") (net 3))
 (segment (start 133.1595 91.3765) (end 133.223 91.313) (width 0.16) (layer "B.Cu") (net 3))
 (segment (start 129.8956 95.4278) (end 136.0551 95.4278) (width 0.16) (layer "F.Cu") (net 1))
 (segment (start 136.0551 95.4278) (end 137.2108 96.5835) (width 0.16) (layer "F.Cu") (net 1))
 (segment (start 129.0066 96.3168) (end 129.2606 96.0628) (width 0.16) (layer "F.Cu") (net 7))
 (segment (start 128.8796 104.9528) (end 128.3716 104.4448) (width 0.16) (layer "F.Cu") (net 7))
 (segment (start 129.326599 104.9528) (end 129.326599 104.586999) (width 0.16) (layer "F.Cu") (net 7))
 (segment (start 129.8956 94.6658) (end 129.8956 93.8288) (width 0.16) (layer "F.Cu") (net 7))
 (segment (start 129.2606 96.0628) (end 129.2606 95.0468) (width 0.16) (layer "F.Cu") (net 7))
 (segment (start 129.2606 95.0468) (end 129.6416 94.6658) (width 0.16) (layer "F.Cu") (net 7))
 (segment (start 129.326599 104.9528) (end 128.8796 104.9528) (width 0.16) (layer "F.Cu") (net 7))
 (segment (start 129.6416 94.6658) (end 129.8956 94.6658) (width 0.16) (layer "F.Cu") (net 7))
 (via (at 128.3716 104.4448) (size 0.8) (drill 0.4) (layers "F.Cu" "B.Cu") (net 7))
 (via (at 129.0066 96.3168) (size 0.8) (drill 0.4) (layers "F.Cu" "B.Cu") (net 7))
 (segment (start 127.7366 104.0638) (end 127.7366 97.3328) (width 0.16) (layer "B.Cu") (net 7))
 (segment (start 128.3716 104.4448) (end 128.1176 104.4448) (width 0.16) (layer "B.Cu") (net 7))
 (segment (start 128.1176 104.4448) (end 127.7366 104.0638) (width 0.16) (layer "B.Cu") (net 7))
 (segment (start 127.7366 97.3328) (end 127.9456 97.1238) (width 0.16) (layer "B.Cu") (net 7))
 (segment (start 127.9456 97.1238) (end 129.0066 96.3168) (width 0.16) (layer "B.Cu") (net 7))
 (segment (start 128.6256 92.6338) (end 128.6256 91.1618) (width 0.16) (layer "F.Cu") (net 10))
 (segment (start 127.8636 93.3958) (end 128.6256 92.6338) (width 0.16) (layer "F.Cu") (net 10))
 (segment (start 127.8636 102.1588) (end 127.8636 93.3958) (width 0.16) (layer "F.Cu") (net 10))
 (segment (start 129.3266 102.4874) (end 128.1922 102.4874) (width 0.16) (layer "F.Cu") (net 10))
 (segment (start 128.1922 102.4874) (end 127.8636 102.1588) (width 0.16) (layer "F.Cu") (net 10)))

